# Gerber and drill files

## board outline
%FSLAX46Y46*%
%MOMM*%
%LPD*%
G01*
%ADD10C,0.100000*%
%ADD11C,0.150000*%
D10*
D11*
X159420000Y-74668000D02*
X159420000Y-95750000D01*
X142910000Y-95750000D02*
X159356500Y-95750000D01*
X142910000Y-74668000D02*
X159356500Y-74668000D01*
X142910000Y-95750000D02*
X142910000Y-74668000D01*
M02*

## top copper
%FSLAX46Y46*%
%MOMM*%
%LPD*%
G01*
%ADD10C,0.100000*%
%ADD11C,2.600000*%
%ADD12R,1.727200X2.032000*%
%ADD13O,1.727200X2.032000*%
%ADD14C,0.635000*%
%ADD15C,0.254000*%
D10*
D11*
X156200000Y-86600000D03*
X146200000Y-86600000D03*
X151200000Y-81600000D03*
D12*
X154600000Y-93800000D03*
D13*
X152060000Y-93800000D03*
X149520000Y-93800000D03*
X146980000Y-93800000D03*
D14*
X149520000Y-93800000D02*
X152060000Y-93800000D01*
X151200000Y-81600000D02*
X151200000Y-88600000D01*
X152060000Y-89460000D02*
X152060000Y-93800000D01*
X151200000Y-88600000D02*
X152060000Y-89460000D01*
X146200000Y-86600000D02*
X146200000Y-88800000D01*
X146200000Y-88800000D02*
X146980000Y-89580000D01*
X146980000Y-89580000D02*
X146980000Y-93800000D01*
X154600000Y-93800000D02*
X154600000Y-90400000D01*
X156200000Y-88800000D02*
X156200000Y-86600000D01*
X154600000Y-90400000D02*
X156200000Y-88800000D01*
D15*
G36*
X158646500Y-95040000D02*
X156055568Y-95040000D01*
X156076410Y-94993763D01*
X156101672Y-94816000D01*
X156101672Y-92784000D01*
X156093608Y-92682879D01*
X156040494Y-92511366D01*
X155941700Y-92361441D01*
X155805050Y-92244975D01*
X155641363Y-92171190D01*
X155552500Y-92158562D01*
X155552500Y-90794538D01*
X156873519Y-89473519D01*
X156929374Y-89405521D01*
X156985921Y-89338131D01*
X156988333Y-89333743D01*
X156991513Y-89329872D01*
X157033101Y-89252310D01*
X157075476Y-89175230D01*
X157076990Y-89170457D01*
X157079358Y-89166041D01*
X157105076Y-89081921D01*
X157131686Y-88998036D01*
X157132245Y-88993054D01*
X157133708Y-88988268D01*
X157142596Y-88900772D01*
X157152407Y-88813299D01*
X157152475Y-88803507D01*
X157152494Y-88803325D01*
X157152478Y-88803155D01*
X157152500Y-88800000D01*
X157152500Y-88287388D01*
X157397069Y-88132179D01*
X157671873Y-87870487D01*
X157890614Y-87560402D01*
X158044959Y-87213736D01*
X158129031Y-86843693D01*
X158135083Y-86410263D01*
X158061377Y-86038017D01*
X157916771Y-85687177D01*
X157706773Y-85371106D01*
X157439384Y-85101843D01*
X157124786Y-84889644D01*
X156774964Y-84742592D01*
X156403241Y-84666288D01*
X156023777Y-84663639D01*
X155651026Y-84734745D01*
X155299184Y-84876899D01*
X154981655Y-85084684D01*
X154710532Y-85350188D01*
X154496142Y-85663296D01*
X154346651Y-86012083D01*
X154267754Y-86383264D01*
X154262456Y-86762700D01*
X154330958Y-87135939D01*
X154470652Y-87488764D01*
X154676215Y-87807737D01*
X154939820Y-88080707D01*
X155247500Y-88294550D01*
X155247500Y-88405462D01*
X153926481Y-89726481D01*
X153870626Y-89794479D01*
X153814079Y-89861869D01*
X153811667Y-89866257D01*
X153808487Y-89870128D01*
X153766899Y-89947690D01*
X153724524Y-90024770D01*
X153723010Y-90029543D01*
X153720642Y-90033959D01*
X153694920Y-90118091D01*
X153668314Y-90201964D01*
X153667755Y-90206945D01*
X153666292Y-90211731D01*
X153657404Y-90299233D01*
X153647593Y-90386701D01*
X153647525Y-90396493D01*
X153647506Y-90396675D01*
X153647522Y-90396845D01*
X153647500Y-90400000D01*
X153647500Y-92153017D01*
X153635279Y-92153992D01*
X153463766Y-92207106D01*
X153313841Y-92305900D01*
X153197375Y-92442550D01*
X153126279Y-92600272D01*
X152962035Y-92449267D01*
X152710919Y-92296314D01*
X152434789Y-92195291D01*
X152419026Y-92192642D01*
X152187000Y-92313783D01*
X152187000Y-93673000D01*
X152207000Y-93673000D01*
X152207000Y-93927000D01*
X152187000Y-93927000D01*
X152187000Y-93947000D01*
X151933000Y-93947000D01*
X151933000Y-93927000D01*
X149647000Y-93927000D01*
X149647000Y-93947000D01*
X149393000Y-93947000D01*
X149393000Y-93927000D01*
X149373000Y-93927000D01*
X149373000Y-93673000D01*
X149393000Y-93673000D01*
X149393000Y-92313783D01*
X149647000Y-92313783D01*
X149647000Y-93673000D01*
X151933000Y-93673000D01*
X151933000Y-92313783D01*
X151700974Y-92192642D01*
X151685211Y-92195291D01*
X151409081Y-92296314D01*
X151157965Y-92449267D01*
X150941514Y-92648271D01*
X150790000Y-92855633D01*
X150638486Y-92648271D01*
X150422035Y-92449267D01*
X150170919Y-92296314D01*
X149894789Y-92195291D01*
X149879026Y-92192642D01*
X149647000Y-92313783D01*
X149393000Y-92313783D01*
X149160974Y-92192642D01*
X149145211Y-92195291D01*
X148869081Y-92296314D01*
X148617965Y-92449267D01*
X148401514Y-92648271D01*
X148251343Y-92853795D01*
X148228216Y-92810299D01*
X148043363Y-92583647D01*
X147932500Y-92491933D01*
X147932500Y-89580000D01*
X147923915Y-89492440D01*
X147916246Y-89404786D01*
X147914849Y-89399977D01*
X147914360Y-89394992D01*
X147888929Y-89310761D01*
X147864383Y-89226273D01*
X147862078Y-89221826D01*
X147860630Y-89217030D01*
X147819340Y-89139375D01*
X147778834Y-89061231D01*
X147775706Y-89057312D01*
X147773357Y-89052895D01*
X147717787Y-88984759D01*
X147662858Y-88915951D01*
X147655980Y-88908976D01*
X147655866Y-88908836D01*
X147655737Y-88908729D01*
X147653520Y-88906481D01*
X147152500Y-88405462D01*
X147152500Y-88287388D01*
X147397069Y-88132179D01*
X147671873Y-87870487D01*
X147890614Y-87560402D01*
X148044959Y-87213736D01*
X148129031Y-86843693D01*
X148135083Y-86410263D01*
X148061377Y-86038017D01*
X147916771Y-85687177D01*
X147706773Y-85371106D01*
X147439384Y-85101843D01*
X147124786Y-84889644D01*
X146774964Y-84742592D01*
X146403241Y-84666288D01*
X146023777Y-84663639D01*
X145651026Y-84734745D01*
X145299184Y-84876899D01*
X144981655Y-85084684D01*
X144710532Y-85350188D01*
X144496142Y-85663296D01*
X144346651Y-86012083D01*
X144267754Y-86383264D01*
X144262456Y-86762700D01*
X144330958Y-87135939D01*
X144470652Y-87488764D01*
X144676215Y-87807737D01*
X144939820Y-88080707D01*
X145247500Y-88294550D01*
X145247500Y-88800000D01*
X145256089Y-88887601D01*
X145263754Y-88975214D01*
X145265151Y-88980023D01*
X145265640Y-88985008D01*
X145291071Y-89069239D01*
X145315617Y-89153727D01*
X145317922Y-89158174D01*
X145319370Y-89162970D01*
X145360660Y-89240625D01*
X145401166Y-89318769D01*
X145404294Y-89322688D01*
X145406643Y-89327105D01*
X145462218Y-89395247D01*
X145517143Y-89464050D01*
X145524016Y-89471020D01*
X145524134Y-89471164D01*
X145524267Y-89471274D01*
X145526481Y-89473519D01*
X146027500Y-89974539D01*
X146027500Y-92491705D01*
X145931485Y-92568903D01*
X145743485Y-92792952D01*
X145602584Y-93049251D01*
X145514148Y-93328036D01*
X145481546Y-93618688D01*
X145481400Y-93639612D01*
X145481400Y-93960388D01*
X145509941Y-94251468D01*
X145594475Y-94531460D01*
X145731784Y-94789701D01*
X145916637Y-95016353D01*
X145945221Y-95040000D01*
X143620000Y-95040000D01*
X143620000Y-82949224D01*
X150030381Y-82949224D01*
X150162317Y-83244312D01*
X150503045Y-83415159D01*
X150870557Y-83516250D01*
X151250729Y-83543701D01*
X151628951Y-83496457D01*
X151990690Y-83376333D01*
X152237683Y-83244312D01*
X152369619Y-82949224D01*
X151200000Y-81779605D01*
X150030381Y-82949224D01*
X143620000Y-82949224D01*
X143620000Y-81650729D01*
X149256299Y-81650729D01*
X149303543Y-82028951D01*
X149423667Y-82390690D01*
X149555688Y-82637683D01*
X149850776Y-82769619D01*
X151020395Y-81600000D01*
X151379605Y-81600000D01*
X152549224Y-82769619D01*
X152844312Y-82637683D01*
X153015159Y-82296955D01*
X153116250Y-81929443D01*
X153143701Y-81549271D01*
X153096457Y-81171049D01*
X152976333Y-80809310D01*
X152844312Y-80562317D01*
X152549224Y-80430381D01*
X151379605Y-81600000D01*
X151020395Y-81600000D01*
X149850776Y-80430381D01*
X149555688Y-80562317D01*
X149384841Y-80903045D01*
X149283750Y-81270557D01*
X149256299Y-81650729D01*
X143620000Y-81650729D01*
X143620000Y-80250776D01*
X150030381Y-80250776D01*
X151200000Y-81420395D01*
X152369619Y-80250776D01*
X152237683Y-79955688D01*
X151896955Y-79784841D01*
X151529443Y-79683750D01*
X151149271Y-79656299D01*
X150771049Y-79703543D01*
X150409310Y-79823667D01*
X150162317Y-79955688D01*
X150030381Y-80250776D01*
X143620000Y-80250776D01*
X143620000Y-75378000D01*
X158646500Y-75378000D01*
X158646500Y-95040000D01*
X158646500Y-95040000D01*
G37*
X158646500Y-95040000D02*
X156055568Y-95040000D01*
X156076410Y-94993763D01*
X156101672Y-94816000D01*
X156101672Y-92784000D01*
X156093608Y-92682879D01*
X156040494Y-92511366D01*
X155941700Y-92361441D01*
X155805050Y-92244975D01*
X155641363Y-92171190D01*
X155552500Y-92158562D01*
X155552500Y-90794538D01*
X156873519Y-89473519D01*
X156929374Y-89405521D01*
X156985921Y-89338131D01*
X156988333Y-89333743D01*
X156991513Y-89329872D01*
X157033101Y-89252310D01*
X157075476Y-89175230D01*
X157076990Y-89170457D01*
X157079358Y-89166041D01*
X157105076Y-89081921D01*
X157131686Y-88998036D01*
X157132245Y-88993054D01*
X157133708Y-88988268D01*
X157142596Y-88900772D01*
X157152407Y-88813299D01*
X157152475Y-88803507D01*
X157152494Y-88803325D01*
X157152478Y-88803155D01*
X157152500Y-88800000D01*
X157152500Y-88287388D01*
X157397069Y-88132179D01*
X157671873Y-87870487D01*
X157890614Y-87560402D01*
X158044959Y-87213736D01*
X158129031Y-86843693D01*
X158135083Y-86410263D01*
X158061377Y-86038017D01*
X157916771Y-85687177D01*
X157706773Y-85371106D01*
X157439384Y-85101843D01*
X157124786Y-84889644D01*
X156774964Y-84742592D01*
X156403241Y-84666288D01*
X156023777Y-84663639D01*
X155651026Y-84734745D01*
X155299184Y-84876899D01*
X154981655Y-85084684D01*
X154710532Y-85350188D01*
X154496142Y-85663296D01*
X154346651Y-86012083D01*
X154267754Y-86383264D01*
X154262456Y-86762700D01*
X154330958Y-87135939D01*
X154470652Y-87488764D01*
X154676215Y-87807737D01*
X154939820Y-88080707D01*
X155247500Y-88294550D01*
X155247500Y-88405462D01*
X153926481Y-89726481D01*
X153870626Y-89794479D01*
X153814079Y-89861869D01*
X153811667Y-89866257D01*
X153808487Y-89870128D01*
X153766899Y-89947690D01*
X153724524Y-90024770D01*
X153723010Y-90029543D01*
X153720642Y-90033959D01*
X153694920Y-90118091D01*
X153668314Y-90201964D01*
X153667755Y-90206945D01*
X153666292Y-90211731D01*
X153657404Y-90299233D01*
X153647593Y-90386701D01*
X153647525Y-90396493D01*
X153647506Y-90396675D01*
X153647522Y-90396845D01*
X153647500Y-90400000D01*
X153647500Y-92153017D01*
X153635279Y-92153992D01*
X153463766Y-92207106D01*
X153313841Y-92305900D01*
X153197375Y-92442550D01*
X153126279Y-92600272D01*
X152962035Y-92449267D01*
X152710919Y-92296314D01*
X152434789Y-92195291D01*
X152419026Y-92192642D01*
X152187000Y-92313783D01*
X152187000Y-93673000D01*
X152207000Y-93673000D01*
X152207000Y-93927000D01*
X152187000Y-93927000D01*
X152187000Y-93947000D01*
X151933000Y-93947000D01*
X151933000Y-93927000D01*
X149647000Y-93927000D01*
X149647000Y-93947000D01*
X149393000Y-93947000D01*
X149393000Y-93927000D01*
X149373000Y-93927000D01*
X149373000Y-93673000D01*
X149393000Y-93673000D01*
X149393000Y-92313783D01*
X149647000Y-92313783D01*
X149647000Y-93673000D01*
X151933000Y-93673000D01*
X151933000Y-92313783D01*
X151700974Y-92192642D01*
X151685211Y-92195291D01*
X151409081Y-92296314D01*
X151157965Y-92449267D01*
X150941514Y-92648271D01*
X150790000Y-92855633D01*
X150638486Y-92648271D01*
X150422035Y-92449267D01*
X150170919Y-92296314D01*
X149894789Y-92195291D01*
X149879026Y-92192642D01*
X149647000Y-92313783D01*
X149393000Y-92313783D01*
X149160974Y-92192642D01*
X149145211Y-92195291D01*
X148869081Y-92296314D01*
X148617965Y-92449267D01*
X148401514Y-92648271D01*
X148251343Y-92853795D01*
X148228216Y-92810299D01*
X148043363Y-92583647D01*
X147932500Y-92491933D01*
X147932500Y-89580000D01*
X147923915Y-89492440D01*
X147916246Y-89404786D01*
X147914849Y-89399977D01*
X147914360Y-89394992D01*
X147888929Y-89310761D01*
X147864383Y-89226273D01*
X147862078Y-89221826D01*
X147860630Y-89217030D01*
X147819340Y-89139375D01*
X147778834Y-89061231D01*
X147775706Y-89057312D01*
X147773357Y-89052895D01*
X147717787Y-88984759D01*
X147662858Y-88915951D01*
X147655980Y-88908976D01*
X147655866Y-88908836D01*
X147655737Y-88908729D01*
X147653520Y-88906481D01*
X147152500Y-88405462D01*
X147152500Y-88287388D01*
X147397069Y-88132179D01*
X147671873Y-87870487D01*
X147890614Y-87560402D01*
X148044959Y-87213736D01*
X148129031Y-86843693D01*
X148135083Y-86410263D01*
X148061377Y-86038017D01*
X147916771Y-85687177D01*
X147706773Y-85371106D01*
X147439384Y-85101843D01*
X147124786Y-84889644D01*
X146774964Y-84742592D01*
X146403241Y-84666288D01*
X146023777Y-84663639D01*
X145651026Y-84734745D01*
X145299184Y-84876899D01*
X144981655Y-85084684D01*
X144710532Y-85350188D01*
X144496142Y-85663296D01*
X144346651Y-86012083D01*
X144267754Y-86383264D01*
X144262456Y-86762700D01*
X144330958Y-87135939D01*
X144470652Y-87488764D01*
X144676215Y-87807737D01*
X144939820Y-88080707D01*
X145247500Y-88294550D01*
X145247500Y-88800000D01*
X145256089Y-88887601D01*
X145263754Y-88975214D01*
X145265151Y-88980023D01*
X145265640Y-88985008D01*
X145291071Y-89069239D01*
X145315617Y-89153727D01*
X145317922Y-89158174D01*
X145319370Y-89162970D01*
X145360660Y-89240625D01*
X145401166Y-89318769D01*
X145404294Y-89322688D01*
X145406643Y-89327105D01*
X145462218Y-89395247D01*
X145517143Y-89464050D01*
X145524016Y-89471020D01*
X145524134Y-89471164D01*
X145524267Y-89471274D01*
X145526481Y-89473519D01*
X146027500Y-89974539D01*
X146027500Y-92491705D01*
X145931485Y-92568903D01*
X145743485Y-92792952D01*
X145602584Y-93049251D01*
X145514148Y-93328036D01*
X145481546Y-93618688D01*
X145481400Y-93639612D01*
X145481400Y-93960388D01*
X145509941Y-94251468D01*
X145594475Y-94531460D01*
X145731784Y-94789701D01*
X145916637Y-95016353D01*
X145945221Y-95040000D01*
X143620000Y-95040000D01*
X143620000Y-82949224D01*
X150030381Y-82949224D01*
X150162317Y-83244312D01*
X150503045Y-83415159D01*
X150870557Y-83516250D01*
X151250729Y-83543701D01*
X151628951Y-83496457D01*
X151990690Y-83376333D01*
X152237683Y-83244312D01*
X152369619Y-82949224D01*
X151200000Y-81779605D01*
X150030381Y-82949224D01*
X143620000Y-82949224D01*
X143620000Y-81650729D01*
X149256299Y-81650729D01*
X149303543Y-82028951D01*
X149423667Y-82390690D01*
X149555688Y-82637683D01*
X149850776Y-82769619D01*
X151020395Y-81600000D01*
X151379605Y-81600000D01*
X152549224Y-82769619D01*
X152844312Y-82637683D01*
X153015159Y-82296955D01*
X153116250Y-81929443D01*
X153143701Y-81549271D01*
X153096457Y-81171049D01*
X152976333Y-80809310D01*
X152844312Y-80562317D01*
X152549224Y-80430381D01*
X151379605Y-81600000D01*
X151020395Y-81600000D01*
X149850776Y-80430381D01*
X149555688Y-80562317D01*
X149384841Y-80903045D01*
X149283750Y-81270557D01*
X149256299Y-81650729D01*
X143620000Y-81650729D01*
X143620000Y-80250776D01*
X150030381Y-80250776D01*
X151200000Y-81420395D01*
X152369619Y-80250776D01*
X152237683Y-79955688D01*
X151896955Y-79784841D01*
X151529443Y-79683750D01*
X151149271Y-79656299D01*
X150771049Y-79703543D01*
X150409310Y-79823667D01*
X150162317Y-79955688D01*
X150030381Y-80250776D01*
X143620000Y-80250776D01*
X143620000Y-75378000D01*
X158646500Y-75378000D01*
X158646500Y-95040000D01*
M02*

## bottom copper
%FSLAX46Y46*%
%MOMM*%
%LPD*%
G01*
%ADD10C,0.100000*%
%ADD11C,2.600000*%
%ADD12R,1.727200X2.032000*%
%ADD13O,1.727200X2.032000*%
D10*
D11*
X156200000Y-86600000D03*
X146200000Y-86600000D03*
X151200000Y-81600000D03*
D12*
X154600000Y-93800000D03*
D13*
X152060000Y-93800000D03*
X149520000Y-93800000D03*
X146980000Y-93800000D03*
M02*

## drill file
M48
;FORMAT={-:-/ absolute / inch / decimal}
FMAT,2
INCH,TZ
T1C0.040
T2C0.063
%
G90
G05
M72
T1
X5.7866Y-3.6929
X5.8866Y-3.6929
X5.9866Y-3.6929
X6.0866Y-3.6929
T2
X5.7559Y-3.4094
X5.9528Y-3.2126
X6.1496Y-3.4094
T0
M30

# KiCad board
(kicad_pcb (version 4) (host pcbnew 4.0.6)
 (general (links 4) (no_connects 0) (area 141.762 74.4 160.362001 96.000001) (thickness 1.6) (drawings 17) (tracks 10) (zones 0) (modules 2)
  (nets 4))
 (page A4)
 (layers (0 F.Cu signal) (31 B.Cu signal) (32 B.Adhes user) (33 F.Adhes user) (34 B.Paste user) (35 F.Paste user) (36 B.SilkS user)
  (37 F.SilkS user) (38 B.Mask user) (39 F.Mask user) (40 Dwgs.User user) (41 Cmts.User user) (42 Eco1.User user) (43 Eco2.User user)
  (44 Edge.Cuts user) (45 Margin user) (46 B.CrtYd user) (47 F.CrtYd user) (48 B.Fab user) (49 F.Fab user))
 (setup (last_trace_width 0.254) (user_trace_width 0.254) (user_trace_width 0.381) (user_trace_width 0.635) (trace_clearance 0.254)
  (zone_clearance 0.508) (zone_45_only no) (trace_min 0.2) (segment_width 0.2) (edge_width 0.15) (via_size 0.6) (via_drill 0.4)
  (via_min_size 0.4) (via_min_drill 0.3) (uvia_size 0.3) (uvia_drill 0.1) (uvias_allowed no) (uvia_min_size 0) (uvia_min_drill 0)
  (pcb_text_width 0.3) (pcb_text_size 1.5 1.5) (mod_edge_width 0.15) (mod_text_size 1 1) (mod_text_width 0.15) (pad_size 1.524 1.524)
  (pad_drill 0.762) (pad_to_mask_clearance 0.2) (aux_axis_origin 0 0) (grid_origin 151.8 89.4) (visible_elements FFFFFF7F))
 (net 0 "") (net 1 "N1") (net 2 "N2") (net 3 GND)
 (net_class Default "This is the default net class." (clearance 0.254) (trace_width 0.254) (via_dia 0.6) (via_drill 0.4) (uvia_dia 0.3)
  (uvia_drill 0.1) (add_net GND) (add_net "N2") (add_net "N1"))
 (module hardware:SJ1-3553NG (layer F.Cu) (at 151.2 84.8 90)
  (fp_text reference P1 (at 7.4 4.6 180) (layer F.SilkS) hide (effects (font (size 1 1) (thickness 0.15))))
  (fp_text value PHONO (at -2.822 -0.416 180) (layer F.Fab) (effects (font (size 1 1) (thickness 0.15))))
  (pad 3 thru_hole circle (at -1.8 5 90) (size 2.6 2.6) (drill 1.6) (layers *.Cu *.Mask F.SilkS) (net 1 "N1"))
  (pad 2 thru_hole circle (at -1.8 -5 90) (size 2.6 2.6) (drill 1.6) (layers *.Cu *.Mask F.SilkS) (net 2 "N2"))
  (pad 1 thru_hole circle (at 3.2 0 90) (size 2.6 2.6) (drill 1.6) (layers *.Cu *.Mask F.SilkS) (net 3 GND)))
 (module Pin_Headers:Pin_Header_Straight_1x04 (layer F.Cu) (at 154.6 93.8 270)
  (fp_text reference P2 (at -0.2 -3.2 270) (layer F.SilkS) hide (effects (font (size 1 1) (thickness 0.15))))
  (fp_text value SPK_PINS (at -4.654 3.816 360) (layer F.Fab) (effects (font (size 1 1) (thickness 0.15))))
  (pad 1 thru_hole rect (at 0 0 270) (size 2.032 1.7272) (drill 1.016) (layers *.Cu *.Mask F.SilkS) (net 1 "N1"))
  (pad 2 thru_hole oval (at 0 2.54 270) (size 2.032 1.7272) (drill 1.016) (layers *.Cu *.Mask F.SilkS) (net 3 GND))
  (pad 3 thru_hole oval (at 0 5.08 270) (size 2.032 1.7272) (drill 1.016) (layers *.Cu *.Mask F.SilkS) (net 3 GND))
  (pad 4 thru_hole oval (at 0 7.62 270) (size 2.032 1.7272) (drill 1.016) (layers *.Cu *.Mask F.SilkS) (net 2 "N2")))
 (gr_line (start 159.42 74.668) (end 159.42 95.75) (angle 90) (layer Edge.Cuts) (width 0.15))
 (gr_line (start 142.91 95.75) (end 159.3565 95.75) (angle 90) (layer Edge.Cuts) (width 0.15))
 (gr_line (start 142.91 74.668) (end 159.3565 74.668) (angle 90) (layer Edge.Cuts) (width 0.15))
 (gr_line (start 142.91 95.75) (end 142.91 74.668) (angle 90) (layer Edge.Cuts) (width 0.15))
 (segment (start 149.52 93.8) (end 152.06 93.8) (width 0.635) (layer F.Cu) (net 3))
 (segment (start 151.2 81.6) (end 151.2 88.6) (width 0.635) (layer F.Cu) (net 3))
 (segment (start 152.06 89.46) (end 152.06 93.8) (width 0.635) (layer F.Cu) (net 3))
 (segment (start 151.2 88.6) (end 152.06 89.46) (width 0.635) (layer F.Cu) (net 3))
 (segment (start 146.2 86.6) (end 146.2 88.8) (width 0.635) (layer F.Cu) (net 2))
 (segment (start 146.2 88.8) (end 146.98 89.58) (width 0.635) (layer F.Cu) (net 2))
 (segment (start 146.98 89.58) (end 146.98 93.8) (width 0.635) (layer F.Cu) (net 2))
 (segment (start 154.6 93.8) (end 154.6 90.4) (width 0.635) (layer F.Cu) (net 1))
 (segment (start 156.2 88.8) (end 156.2 86.6) (width 0.635) (layer F.Cu) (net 1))
 (segment (start 154.6 90.4) (end 156.2 88.8) (width 0.635) (layer F.Cu) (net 1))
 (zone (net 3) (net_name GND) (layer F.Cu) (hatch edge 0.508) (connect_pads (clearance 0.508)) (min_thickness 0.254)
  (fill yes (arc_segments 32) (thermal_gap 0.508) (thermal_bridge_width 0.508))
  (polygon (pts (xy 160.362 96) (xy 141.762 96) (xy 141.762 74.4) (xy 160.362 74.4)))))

